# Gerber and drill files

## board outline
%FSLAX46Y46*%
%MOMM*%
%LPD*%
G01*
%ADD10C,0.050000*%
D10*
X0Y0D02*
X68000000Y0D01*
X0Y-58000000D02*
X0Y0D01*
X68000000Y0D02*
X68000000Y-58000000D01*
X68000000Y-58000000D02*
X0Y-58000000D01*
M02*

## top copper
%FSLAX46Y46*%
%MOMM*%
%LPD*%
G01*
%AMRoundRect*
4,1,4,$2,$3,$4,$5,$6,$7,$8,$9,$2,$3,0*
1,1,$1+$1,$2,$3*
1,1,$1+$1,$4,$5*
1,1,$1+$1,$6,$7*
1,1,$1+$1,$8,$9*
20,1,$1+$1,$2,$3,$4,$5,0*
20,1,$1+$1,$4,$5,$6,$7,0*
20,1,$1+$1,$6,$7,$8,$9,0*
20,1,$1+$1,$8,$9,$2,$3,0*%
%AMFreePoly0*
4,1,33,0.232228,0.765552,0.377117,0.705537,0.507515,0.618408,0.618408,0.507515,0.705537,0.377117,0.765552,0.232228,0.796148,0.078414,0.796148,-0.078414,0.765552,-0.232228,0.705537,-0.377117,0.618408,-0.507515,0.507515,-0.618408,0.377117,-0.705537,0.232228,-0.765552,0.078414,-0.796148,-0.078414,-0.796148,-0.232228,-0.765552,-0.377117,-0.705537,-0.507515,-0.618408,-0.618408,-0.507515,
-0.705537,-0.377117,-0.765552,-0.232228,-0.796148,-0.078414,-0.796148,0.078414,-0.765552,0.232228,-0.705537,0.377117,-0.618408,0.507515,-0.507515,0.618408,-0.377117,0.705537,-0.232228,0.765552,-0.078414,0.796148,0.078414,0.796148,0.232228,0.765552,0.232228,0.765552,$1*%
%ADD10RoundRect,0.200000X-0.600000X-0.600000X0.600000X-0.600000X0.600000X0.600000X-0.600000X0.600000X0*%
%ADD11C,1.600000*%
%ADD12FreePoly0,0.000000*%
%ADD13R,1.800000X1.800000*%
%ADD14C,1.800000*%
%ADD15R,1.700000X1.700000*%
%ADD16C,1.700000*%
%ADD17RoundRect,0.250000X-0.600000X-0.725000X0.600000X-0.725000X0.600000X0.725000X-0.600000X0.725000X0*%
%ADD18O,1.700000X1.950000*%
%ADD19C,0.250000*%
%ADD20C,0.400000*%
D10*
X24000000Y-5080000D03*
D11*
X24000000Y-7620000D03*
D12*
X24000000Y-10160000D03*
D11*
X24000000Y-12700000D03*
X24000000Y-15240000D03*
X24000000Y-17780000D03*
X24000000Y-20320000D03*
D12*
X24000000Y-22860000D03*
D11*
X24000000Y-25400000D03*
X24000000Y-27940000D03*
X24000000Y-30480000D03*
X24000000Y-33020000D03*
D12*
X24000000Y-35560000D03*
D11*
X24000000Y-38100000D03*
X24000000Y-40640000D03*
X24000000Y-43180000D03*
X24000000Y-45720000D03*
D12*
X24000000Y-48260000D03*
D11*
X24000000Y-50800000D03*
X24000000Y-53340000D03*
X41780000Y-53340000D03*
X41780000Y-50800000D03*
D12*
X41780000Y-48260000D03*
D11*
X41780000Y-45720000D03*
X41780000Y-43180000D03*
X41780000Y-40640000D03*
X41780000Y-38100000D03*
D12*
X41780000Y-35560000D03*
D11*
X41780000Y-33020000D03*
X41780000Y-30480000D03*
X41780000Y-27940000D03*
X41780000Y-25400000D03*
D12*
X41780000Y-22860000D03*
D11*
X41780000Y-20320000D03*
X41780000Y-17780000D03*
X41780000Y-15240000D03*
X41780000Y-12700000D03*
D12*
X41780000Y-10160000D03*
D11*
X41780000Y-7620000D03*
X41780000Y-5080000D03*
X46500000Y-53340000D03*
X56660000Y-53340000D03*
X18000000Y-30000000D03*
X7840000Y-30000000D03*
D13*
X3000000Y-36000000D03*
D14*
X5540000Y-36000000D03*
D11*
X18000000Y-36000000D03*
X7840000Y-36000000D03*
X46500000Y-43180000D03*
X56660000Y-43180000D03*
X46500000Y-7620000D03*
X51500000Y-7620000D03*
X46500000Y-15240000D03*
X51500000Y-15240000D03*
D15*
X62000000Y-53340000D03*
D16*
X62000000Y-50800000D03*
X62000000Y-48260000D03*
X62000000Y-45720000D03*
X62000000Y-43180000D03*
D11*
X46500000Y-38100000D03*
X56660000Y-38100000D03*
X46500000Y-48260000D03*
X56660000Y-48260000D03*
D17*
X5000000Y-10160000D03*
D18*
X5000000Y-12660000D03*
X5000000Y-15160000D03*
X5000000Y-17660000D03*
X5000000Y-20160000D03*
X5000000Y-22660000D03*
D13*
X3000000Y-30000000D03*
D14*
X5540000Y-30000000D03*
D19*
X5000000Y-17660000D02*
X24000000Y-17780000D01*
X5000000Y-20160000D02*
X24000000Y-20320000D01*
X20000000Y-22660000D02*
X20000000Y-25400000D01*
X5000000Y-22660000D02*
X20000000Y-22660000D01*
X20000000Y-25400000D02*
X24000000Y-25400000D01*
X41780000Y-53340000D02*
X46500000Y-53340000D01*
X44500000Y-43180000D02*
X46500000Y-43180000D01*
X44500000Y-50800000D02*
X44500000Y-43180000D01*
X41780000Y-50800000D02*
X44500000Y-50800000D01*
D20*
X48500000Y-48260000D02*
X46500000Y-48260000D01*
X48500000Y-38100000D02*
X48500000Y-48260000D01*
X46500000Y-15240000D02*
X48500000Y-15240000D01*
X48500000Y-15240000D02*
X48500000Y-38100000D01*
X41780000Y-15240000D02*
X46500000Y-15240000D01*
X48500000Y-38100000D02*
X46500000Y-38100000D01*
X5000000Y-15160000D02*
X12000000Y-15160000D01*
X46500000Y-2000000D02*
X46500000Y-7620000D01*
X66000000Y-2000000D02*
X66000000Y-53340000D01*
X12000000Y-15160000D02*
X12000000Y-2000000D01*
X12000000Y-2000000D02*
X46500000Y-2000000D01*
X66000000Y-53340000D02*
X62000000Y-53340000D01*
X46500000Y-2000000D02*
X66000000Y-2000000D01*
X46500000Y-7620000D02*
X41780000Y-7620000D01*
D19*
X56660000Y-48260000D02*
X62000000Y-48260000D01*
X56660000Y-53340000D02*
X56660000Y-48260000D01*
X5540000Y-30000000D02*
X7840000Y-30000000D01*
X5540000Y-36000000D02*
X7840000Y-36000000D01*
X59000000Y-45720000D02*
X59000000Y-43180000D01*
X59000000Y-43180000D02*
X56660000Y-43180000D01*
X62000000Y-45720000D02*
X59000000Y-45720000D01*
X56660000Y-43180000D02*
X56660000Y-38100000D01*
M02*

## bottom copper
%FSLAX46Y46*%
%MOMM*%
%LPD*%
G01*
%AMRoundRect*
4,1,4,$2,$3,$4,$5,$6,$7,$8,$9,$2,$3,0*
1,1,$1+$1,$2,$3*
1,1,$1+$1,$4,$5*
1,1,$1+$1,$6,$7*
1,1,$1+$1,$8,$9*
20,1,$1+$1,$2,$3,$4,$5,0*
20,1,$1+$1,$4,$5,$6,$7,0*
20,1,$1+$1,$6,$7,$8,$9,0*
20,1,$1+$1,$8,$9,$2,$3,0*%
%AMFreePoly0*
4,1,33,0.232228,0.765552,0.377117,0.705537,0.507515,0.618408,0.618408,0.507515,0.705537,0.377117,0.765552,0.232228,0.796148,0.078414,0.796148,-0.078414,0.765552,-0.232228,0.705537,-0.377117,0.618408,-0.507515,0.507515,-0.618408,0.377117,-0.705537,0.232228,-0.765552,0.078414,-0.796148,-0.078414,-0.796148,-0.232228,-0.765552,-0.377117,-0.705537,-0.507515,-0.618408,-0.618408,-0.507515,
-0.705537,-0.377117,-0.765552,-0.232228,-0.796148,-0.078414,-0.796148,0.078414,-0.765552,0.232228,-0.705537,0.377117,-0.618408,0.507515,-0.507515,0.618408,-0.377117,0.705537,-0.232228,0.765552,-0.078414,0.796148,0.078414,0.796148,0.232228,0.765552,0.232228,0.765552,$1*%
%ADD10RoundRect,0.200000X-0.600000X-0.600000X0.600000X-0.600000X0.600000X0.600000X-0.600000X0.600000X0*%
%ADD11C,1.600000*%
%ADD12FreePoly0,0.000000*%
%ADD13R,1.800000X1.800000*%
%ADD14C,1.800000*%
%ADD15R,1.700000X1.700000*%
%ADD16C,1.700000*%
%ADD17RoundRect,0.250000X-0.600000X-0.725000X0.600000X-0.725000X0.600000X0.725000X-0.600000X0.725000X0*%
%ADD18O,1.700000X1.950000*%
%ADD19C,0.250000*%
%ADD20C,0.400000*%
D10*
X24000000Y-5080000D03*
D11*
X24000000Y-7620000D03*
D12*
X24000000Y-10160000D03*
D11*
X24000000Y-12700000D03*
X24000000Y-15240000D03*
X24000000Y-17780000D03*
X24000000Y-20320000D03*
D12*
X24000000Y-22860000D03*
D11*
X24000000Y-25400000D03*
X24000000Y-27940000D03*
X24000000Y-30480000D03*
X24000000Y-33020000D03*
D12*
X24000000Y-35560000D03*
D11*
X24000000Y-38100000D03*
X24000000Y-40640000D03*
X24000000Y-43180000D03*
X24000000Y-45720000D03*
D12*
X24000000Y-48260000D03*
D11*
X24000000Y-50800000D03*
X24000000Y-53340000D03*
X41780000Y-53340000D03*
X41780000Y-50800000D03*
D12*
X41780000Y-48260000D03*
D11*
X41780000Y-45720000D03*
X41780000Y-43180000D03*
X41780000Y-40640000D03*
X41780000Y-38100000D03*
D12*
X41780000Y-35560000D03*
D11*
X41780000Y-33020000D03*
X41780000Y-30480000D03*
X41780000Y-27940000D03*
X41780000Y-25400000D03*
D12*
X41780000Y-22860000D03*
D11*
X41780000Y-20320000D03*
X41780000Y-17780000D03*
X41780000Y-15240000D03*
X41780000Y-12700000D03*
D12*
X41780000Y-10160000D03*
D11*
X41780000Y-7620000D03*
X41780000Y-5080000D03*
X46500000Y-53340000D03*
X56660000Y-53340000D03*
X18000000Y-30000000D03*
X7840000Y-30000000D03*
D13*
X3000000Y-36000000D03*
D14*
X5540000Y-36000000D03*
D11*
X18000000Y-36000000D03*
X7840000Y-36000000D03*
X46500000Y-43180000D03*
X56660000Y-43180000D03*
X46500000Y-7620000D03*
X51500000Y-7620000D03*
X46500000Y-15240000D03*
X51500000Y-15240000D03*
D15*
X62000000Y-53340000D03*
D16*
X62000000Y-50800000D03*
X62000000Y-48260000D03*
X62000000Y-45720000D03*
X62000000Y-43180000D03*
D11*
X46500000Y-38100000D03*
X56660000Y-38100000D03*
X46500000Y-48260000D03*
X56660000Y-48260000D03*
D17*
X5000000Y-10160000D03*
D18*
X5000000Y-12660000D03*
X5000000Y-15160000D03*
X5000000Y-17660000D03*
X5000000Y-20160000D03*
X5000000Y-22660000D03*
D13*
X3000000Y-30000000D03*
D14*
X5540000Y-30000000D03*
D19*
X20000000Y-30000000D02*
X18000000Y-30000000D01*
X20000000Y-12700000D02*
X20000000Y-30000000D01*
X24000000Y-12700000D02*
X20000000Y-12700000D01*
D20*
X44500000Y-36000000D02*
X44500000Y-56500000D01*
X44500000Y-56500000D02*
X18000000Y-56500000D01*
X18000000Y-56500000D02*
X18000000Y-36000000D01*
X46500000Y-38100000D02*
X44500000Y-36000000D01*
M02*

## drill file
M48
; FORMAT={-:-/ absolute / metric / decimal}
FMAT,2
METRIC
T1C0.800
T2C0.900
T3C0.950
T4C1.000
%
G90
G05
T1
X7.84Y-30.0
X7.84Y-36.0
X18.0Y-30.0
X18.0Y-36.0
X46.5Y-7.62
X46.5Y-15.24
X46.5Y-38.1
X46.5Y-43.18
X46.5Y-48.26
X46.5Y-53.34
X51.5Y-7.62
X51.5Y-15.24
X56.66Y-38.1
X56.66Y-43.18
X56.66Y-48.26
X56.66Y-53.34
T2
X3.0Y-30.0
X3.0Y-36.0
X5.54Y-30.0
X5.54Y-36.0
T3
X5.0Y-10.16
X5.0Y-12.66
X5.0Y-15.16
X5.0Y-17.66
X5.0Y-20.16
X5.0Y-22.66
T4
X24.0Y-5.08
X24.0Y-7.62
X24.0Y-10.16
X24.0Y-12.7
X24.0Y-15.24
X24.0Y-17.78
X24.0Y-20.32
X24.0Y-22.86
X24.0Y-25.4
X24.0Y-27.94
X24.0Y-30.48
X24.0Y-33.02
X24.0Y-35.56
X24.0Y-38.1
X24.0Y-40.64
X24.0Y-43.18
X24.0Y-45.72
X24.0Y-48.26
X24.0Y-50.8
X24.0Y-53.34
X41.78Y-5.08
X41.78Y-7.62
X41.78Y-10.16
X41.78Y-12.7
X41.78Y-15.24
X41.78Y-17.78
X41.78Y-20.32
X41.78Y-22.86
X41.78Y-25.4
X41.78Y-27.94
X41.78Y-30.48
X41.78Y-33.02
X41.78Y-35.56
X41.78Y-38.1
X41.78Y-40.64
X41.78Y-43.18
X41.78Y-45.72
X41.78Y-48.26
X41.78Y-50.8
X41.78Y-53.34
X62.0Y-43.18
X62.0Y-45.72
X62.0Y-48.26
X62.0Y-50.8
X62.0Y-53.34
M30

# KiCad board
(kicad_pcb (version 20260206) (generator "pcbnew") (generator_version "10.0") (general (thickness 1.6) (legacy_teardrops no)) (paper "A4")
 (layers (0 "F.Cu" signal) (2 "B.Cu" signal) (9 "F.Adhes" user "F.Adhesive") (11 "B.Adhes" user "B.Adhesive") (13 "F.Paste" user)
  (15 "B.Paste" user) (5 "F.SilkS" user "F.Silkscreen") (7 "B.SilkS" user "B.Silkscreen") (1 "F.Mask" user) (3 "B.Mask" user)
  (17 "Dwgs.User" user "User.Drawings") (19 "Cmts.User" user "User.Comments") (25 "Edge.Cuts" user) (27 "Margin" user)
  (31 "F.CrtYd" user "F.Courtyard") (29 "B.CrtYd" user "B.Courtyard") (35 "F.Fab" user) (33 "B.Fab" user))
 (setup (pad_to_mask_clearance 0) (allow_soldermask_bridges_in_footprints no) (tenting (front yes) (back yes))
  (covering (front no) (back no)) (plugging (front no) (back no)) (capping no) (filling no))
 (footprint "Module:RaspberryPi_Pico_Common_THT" (layer "F.Cu") (at 24 5.08)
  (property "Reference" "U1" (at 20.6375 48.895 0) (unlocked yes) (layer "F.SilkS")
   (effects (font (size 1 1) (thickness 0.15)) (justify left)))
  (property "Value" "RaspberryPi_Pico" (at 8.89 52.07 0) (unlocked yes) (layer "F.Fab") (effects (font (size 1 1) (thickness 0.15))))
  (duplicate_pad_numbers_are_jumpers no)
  (pad "1" thru_hole roundrect (at 0 0) (size 1.6 1.6) (drill 1) (layers "*.Cu" "*.Mask") (remove_unused_layers no) (roundrect_rratio 0.125)
   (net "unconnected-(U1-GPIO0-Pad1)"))
  (pad "2" thru_hole circle (at 0 2.54) (size 1.6 1.6) (drill 1) (layers "*.Cu" "*.Mask") (remove_unused_layers no)
   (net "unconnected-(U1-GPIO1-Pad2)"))
  (pad "3" thru_hole custom (at 0 5.08) (size 1.6 1.6) (drill 1) (layers "*.Cu" "*.Mask") (remove_unused_layers no) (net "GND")
   (options (clearance outline) (anchor circle)) (primitives))
  (pad "4" thru_hole circle (at 0 7.62) (size 1.6 1.6) (drill 1) (layers "*.Cu" "*.Mask") (remove_unused_layers no) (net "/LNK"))
  (pad "5" thru_hole circle (at 0 10.16) (size 1.6 1.6) (drill 1) (layers "*.Cu" "*.Mask") (remove_unused_layers no)
   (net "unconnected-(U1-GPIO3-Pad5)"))
  (pad "6" thru_hole circle (at 0 12.7) (size 1.6 1.6) (drill 1) (layers "*.Cu" "*.Mask") (remove_unused_layers no) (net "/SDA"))
  (pad "7" thru_hole circle (at 0 15.24) (size 1.6 1.6) (drill 1) (layers "*.Cu" "*.Mask") (remove_unused_layers no) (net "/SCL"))
  (pad "8" thru_hole custom (at 0 17.78) (size 1.6 1.6) (drill 1) (layers "*.Cu" "*.Mask") (remove_unused_layers no) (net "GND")
   (options (clearance outline) (anchor circle)) (primitives))
  (pad "9" thru_hole circle (at 0 20.32) (size 1.6 1.6) (drill 1) (layers "*.Cu" "*.Mask") (remove_unused_layers no) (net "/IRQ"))
  (pad "10" thru_hole circle (at 0 22.86) (size 1.6 1.6) (drill 1) (layers "*.Cu" "*.Mask") (remove_unused_layers no)
   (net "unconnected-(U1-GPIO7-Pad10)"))
  (pad "11" thru_hole circle (at 0 25.4) (size 1.6 1.6) (drill 1) (layers "*.Cu" "*.Mask") (remove_unused_layers no)
   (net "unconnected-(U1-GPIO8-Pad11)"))
  (pad "12" thru_hole circle (at 0 27.94) (size 1.6 1.6) (drill 1) (layers "*.Cu" "*.Mask") (remove_unused_layers no)
   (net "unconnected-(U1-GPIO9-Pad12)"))
  (pad "13" thru_hole custom (at 0 30.48) (size 1.6 1.6) (drill 1) (layers "*.Cu" "*.Mask") (remove_unused_layers no) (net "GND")
   (options (clearance outline) (anchor circle)) (primitives))
  (pad "14" thru_hole circle (at 0 33.02) (size 1.6 1.6) (drill 1) (layers "*.Cu" "*.Mask") (remove_unused_layers no)
   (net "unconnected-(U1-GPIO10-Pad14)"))
  (pad "15" thru_hole circle (at 0 35.56) (size 1.6 1.6) (drill 1) (layers "*.Cu" "*.Mask") (remove_unused_layers no)
   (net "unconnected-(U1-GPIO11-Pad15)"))
  (pad "16" thru_hole circle (at 0 38.1) (size 1.6 1.6) (drill 1) (layers "*.Cu" "*.Mask") (remove_unused_layers no)
   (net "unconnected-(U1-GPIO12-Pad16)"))
  (pad "17" thru_hole circle (at 0 40.64) (size 1.6 1.6) (drill 1) (layers "*.Cu" "*.Mask") (remove_unused_layers no)
   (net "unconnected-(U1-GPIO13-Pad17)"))
  (pad "18" thru_hole custom (at 0 43.18) (size 1.6 1.6) (drill 1) (layers "*.Cu" "*.Mask") (remove_unused_layers no) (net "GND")
   (options (clearance outline) (anchor circle)) (primitives))
  (pad "19" thru_hole circle (at 0 45.72) (size 1.6 1.6) (drill 1) (layers "*.Cu" "*.Mask") (remove_unused_layers no)
   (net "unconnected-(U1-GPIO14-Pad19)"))
  (pad "20" thru_hole circle (at 0 48.26) (size 1.6 1.6) (drill 1) (layers "*.Cu" "*.Mask") (remove_unused_layers no)
   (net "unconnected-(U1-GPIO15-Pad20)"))
  (pad "21" thru_hole circle (at 17.78 48.26) (size 1.6 1.6) (drill 1) (layers "*.Cu" "*.Mask") (remove_unused_layers no) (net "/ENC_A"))
  (pad "22" thru_hole circle (at 17.78 45.72) (size 1.6 1.6) (drill 1) (layers "*.Cu" "*.Mask") (remove_unused_layers no) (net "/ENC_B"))
  (pad "23" thru_hole custom (at 17.78 43.18) (size 1.6 1.6) (drill 1) (layers "*.Cu" "*.Mask") (remove_unused_layers no) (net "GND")
   (options (clearance outline) (anchor circle)) (primitives))
  (pad "24" thru_hole circle (at 17.78 40.64) (size 1.6 1.6) (drill 1) (layers "*.Cu" "*.Mask") (remove_unused_layers no)
   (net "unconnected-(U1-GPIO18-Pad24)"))
  (pad "25" thru_hole circle (at 17.78 38.1) (size 1.6 1.6) (drill 1) (layers "*.Cu" "*.Mask") (remove_unused_layers no)
   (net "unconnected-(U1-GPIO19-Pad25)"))
  (pad "26" thru_hole circle (at 17.78 35.56) (size 1.6 1.6) (drill 1) (layers "*.Cu" "*.Mask") (remove_unused_layers no)
   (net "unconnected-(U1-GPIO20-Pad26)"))
  (pad "27" thru_hole circle (at 17.78 33.02) (size 1.6 1.6) (drill 1) (layers "*.Cu" "*.Mask") (remove_unused_layers no)
   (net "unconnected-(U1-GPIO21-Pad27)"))
  (pad "28" thru_hole custom (at 17.78 30.48) (size 1.6 1.6) (drill 1) (layers "*.Cu" "*.Mask") (remove_unused_layers no) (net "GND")
   (options (clearance outline) (anchor circle)) (primitives))
  (pad "29" thru_hole circle (at 17.78 27.94) (size 1.6 1.6) (drill 1) (layers "*.Cu" "*.Mask") (remove_unused_layers no)
   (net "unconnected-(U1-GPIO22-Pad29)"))
  (pad "30" thru_hole circle (at 17.78 25.4) (size 1.6 1.6) (drill 1) (layers "*.Cu" "*.Mask") (remove_unused_layers no)
   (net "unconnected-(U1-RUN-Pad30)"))
  (pad "31" thru_hole circle (at 17.78 22.86) (size 1.6 1.6) (drill 1) (layers "*.Cu" "*.Mask") (remove_unused_layers no)
   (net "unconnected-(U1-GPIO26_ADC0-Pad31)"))
  (pad "32" thru_hole circle (at 17.78 20.32) (size 1.6 1.6) (drill 1) (layers "*.Cu" "*.Mask") (remove_unused_layers no)
   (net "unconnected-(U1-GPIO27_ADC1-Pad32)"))
  (pad "33" thru_hole custom (at 17.78 17.78) (size 1.6 1.6) (drill 1) (layers "*.Cu" "*.Mask") (remove_unused_layers no)
   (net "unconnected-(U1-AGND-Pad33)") (options (clearance outline) (anchor circle)) (primitives))
  (pad "34" thru_hole circle (at 17.78 15.24) (size 1.6 1.6) (drill 1) (layers "*.Cu" "*.Mask") (remove_unused_layers no)
   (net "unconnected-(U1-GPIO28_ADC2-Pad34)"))
  (pad "35" thru_hole circle (at 17.78 12.7) (size 1.6 1.6) (drill 1) (layers "*.Cu" "*.Mask") (remove_unused_layers no)
   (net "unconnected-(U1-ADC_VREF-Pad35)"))
  (pad "36" thru_hole circle (at 17.78 10.16) (size 1.6 1.6) (drill 1) (layers "*.Cu" "*.Mask") (remove_unused_layers no) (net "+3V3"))
  (pad "37" thru_hole circle (at 17.78 7.62) (size 1.6 1.6) (drill 1) (layers "*.Cu" "*.Mask") (remove_unused_layers no)
   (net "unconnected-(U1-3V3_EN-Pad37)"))
  (pad "38" thru_hole custom (at 17.78 5.08) (size 1.6 1.6) (drill 1) (layers "*.Cu" "*.Mask") (remove_unused_layers no) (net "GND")
   (options (clearance outline) (anchor circle)) (primitives))
  (pad "39" thru_hole circle (at 17.78 2.54) (size 1.6 1.6) (drill 1) (layers "*.Cu" "*.Mask") (remove_unused_layers no) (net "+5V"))
  (pad "40" thru_hole circle (at 17.78 0) (size 1.6 1.6) (drill 1) (layers "*.Cu" "*.Mask") (remove_unused_layers no)
   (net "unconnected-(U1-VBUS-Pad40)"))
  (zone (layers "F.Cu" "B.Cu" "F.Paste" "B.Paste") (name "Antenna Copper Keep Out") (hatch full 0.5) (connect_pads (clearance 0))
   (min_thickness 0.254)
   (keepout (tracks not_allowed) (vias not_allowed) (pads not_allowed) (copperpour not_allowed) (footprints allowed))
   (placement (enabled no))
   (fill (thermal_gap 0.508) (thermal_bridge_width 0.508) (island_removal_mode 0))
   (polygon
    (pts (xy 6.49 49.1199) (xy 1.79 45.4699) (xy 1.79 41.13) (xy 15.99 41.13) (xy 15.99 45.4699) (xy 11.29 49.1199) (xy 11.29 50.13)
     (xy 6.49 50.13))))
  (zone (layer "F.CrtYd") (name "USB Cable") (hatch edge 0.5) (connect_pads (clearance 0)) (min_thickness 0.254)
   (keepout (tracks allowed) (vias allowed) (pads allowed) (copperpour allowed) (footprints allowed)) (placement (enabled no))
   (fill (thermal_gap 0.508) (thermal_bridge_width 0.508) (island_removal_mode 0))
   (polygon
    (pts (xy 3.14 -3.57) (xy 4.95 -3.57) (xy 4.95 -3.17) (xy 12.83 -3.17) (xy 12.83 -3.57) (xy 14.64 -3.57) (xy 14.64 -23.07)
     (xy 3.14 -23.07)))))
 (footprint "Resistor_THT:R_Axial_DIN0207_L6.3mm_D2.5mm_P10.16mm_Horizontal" (layer "F.Cu") (at 46.5 53.34)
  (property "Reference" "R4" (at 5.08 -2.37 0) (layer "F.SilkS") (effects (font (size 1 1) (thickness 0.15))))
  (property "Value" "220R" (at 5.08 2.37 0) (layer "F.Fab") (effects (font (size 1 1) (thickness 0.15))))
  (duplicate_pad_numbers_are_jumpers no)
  (pad "1" thru_hole circle (at 0 0) (size 1.6 1.6) (drill 0.8) (layers "*.Cu" "*.Mask") (remove_unused_layers no) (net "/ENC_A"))
  (pad "2" thru_hole circle (at 10.16 0) (size 1.6 1.6) (drill 0.8) (layers "*.Cu" "*.Mask") (remove_unused_layers no) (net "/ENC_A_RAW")))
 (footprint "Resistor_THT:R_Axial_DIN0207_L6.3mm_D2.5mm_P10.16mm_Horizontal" (layer "F.Cu") (at 18 30 180)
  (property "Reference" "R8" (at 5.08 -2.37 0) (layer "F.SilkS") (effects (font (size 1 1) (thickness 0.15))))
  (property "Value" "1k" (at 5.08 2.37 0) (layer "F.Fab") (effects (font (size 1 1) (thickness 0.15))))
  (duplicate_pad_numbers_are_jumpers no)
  (pad "1" thru_hole circle (at 0 0) (size 1.6 1.6) (drill 0.8) (layers "*.Cu" "*.Mask") (remove_unused_layers no) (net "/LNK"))
  (pad "2" thru_hole circle (at 10.16 0) (size 1.6 1.6) (drill 0.8) (layers "*.Cu" "*.Mask") (remove_unused_layers no) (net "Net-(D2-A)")))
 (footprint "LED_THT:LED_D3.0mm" (layer "F.Cu") (at 3 36)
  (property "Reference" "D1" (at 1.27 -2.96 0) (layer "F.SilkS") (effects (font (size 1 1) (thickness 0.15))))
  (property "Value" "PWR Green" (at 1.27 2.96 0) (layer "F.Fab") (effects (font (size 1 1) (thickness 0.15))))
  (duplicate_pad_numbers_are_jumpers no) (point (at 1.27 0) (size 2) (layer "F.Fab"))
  (pad "1" thru_hole rect (at 0 0) (size 1.8 1.8) (drill 0.9) (layers "*.Cu" "*.Mask") (remove_unused_layers no) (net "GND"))
  (pad "2" thru_hole circle (at 2.54 0) (size 1.8 1.8) (drill 0.9) (layers "*.Cu" "*.Mask") (remove_unused_layers no) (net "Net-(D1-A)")))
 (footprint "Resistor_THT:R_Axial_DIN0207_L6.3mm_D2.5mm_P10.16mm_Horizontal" (layer "F.Cu") (at 18 36 180)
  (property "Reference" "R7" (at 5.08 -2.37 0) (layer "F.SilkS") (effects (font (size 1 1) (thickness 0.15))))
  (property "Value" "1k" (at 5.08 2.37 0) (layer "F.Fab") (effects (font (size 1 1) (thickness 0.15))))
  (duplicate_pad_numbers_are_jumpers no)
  (pad "1" thru_hole circle (at 0 0) (size 1.6 1.6) (drill 0.8) (layers "*.Cu" "*.Mask") (remove_unused_layers no) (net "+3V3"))
  (pad "2" thru_hole circle (at 10.16 0) (size 1.6 1.6) (drill 0.8) (layers "*.Cu" "*.Mask") (remove_unused_layers no) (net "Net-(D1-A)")))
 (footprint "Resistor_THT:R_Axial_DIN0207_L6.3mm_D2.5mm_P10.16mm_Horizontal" (layer "F.Cu") (at 46.5 43.18)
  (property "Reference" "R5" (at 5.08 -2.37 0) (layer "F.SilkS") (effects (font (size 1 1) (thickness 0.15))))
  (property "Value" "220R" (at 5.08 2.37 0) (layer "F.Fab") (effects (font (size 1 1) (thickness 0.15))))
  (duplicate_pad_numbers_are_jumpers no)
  (pad "1" thru_hole circle (at 0 0) (size 1.6 1.6) (drill 0.8) (layers "*.Cu" "*.Mask") (remove_unused_layers no) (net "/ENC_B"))
  (pad "2" thru_hole circle (at 10.16 0) (size 1.6 1.6) (drill 0.8) (layers "*.Cu" "*.Mask") (remove_unused_layers no) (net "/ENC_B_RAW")))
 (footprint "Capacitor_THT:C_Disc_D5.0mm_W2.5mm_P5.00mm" (layer "F.Cu") (at 46.5 7.62)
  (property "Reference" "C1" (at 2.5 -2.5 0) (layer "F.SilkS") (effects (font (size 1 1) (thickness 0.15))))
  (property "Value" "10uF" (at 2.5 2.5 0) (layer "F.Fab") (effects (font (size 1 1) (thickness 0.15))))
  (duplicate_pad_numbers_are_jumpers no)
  (pad "1" thru_hole circle (at 0 0) (size 1.6 1.6) (drill 0.8) (layers "*.Cu" "*.Mask") (remove_unused_layers no) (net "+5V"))
  (pad "2" thru_hole circle (at 5 0) (size 1.6 1.6) (drill 0.8) (layers "*.Cu" "*.Mask") (remove_unused_layers no) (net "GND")))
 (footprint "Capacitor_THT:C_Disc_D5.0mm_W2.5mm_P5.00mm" (layer "F.Cu") (at 46.5 15.24)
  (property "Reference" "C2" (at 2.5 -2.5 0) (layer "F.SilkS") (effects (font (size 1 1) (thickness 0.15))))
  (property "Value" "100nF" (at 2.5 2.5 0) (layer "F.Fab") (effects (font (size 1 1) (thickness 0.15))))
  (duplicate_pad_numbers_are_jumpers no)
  (pad "1" thru_hole circle (at 0 0) (size 1.6 1.6) (drill 0.8) (layers "*.Cu" "*.Mask") (remove_unused_layers no) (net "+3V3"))
  (pad "2" thru_hole circle (at 5 0) (size 1.6 1.6) (drill 0.8) (layers "*.Cu" "*.Mask") (remove_unused_layers no) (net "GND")))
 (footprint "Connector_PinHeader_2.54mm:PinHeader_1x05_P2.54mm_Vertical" (layer "F.Cu") (at 62 53.34 180)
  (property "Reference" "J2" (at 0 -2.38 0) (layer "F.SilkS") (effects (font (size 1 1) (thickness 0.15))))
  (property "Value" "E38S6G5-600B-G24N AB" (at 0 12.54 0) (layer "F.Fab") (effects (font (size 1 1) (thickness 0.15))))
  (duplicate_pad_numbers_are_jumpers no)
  (pad "1" thru_hole rect (at 0 0) (size 1.7 1.7) (drill 1) (layers "*.Cu" "*.Mask") (remove_unused_layers no) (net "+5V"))
  (pad "2" thru_hole circle (at 0 2.54) (size 1.7 1.7) (drill 1) (layers "*.Cu" "*.Mask") (remove_unused_layers no) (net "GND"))
  (pad "3" thru_hole circle (at 0 5.08) (size 1.7 1.7) (drill 1) (layers "*.Cu" "*.Mask") (remove_unused_layers no) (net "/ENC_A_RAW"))
  (pad "4" thru_hole circle (at 0 7.62) (size 1.7 1.7) (drill 1) (layers "*.Cu" "*.Mask") (remove_unused_layers no) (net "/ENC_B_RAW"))
  (pad "5" thru_hole circle (at 0 10.16) (size 1.7 1.7) (drill 1) (layers "*.Cu" "*.Mask") (remove_unused_layers no) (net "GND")))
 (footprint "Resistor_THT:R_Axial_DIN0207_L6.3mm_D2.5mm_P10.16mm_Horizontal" (layer "F.Cu") (at 46.5 38.1)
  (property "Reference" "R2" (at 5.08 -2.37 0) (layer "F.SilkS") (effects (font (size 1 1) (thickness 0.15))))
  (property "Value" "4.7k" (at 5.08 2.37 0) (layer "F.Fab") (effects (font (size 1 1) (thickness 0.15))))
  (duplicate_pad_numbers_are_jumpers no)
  (pad "1" thru_hole circle (at 0 0) (size 1.6 1.6) (drill 0.8) (layers "*.Cu" "*.Mask") (remove_unused_layers no) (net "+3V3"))
  (pad "2" thru_hole circle (at 10.16 0) (size 1.6 1.6) (drill 0.8) (layers "*.Cu" "*.Mask") (remove_unused_layers no) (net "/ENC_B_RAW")))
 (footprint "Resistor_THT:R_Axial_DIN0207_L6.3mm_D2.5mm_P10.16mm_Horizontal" (layer "F.Cu") (at 46.5 48.26)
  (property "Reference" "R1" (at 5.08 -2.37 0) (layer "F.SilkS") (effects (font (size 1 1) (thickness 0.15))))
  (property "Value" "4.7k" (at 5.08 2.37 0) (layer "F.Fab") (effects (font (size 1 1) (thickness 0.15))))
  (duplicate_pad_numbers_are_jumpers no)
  (pad "1" thru_hole circle (at 0 0) (size 1.6 1.6) (drill 0.8) (layers "*.Cu" "*.Mask") (remove_unused_layers no) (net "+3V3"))
  (pad "2" thru_hole circle (at 10.16 0) (size 1.6 1.6) (drill 0.8) (layers "*.Cu" "*.Mask") (remove_unused_layers no) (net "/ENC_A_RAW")))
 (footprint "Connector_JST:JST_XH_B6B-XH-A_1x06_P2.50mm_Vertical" (layer "F.Cu") (at 5 10.16 -90)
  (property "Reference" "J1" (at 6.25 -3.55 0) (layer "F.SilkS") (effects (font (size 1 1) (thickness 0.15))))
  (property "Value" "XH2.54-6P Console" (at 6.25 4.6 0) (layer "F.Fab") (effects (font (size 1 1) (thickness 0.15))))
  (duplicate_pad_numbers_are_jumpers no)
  (pad "1" thru_hole roundrect (at 0 0) (size 1.7 1.95) (drill 0.95) (layers "*.Cu" "*.Mask") (remove_unused_layers no)
   (roundrect_rratio 0.147059) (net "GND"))
  (pad "2" thru_hole oval (at 2.5 0) (size 1.7 1.95) (drill 0.95) (layers "*.Cu" "*.Mask") (remove_unused_layers no)
   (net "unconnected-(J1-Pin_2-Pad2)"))
  (pad "3" thru_hole oval (at 5 0) (size 1.7 1.95) (drill 0.95) (layers "*.Cu" "*.Mask") (remove_unused_layers no) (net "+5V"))
  (pad "4" thru_hole oval (at 7.5 0) (size 1.7 1.95) (drill 0.95) (layers "*.Cu" "*.Mask") (remove_unused_layers no) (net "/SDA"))
  (pad "5" thru_hole oval (at 10 0) (size 1.7 1.95) (drill 0.95) (layers "*.Cu" "*.Mask") (remove_unused_layers no) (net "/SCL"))
  (pad "6" thru_hole oval (at 12.5 0) (size 1.7 1.95) (drill 0.95) (layers "*.Cu" "*.Mask") (remove_unused_layers no) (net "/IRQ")))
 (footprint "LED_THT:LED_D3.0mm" (layer "F.Cu") (at 3 30)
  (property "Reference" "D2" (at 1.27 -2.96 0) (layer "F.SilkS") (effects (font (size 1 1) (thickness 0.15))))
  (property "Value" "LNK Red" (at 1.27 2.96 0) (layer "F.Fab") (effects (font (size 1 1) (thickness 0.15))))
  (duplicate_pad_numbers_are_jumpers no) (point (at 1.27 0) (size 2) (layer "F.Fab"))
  (pad "1" thru_hole rect (at 0 0) (size 1.8 1.8) (drill 0.9) (layers "*.Cu" "*.Mask") (remove_unused_layers no) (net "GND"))
  (pad "2" thru_hole circle (at 2.54 0) (size 1.8 1.8) (drill 0.9) (layers "*.Cu" "*.Mask") (remove_unused_layers no) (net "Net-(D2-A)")))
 (gr_line (start 0 0) (end 68 0) (stroke (width 0.05) (type solid)) (layer "Edge.Cuts"))
 (gr_line (start 0 58) (end 0 0) (stroke (width 0.05) (type solid)) (layer "Edge.Cuts"))
 (gr_line (start 68 0) (end 68 58) (stroke (width 0.05) (type solid)) (layer "Edge.Cuts"))
 (gr_line (start 68 58) (end 0 58) (stroke (width 0.05) (type solid)) (layer "Edge.Cuts"))
 (segment (start 20 30) (end 18 30) (width 0.25) (layer "B.Cu") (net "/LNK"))
 (segment (start 20 12.7) (end 20 30) (width 0.25) (layer "B.Cu") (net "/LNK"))
 (segment (start 24 12.7) (end 20 12.7) (width 0.25) (layer "B.Cu") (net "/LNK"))
 (segment (start 5 17.66) (end 24 17.78) (width 0.25) (layer "F.Cu") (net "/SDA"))
 (segment (start 5 20.16) (end 24 20.32) (width 0.25) (layer "F.Cu") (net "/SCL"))
 (segment (start 20 22.66) (end 20 25.4) (width 0.25) (layer "F.Cu") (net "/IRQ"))
 (segment (start 5 22.66) (end 20 22.66) (width 0.25) (layer "F.Cu") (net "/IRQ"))
 (segment (start 20 25.4) (end 24 25.4) (width 0.25) (layer "F.Cu") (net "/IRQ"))
 (segment (start 41.78 53.34) (end 46.5 53.34) (width 0.25) (layer "F.Cu") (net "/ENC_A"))
 (segment (start 44.5 43.18) (end 46.5 43.18) (width 0.25) (layer "F.Cu") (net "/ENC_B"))
 (segment (start 44.5 50.8) (end 44.5 43.18) (width 0.25) (layer "F.Cu") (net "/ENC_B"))
 (segment (start 41.78 50.8) (end 44.5 50.8) (width 0.25) (layer "F.Cu") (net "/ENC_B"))
 (segment (start 48.5 48.26) (end 46.5 48.26) (width 0.4) (layer "F.Cu") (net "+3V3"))
 (segment (start 48.5 38.1) (end 48.5 48.26) (width 0.4) (layer "F.Cu") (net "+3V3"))
 (segment (start 46.5 15.24) (end 48.5 15.24) (width 0.4) (layer "F.Cu") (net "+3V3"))
 (segment (start 48.5 15.24) (end 48.5 38.1) (width 0.4) (layer "F.Cu") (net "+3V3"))
 (segment (start 41.78 15.24) (end 46.5 15.24) (width 0.4) (layer "F.Cu") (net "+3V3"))
 (segment (start 48.5 38.1) (end 46.5 38.1) (width 0.4) (layer "F.Cu") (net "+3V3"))
 (segment (start 44.5 36) (end 44.5 56.5) (width 0.4) (layer "B.Cu") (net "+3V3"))
 (segment (start 44.5 56.5) (end 18 56.5) (width 0.4) (layer "B.Cu") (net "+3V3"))
 (segment (start 18 56.5) (end 18 36) (width 0.4) (layer "B.Cu") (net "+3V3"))
 (segment (start 46.5 38.1) (end 44.5 36) (width 0.4) (layer "B.Cu") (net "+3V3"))
 (segment (start 5 15.16) (end 12 15.16) (width 0.4) (layer "F.Cu") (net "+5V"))
 (segment (start 46.5 2) (end 46.5 7.62) (width 0.4) (layer "F.Cu") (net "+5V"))
 (segment (start 66 2) (end 66 53.34) (width 0.4) (layer "F.Cu") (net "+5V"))
 (segment (start 12 15.16) (end 12 2) (width 0.4) (layer "F.Cu") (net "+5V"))
 (segment (start 12 2) (end 46.5 2) (width 0.4) (layer "F.Cu") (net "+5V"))
 (segment (start 66 53.34) (end 62 53.34) (width 0.4) (layer "F.Cu") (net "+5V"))
 (segment (start 46.5 2) (end 66 2) (width 0.4) (layer "F.Cu") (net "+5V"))
 (segment (start 46.5 7.62) (end 41.78 7.62) (width 0.4) (layer "F.Cu") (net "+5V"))
 (segment (start 56.66 48.26) (end 62 48.26) (width 0.25) (layer "F.Cu") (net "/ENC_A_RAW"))
 (segment (start 56.66 53.34) (end 56.66 48.26) (width 0.25) (layer "F.Cu") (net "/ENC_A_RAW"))
 (segment (start 5.54 30) (end 7.84 30) (width 0.25) (layer "F.Cu") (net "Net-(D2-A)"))
 (segment (start 5.54 36) (end 7.84 36) (width 0.25) (layer "F.Cu") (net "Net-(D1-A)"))
 (segment (start 59 45.72) (end 59 43.18) (width 0.25) (layer "F.Cu") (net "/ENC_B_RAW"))
 (segment (start 59 43.18) (end 56.66 43.18) (width 0.25) (layer "F.Cu") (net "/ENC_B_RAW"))
 (segment (start 62 45.72) (end 59 45.72) (width 0.25) (layer "F.Cu") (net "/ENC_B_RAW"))
 (segment (start 56.66 43.18) (end 56.66 38.1) (width 0.25) (layer "F.Cu") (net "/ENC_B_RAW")))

